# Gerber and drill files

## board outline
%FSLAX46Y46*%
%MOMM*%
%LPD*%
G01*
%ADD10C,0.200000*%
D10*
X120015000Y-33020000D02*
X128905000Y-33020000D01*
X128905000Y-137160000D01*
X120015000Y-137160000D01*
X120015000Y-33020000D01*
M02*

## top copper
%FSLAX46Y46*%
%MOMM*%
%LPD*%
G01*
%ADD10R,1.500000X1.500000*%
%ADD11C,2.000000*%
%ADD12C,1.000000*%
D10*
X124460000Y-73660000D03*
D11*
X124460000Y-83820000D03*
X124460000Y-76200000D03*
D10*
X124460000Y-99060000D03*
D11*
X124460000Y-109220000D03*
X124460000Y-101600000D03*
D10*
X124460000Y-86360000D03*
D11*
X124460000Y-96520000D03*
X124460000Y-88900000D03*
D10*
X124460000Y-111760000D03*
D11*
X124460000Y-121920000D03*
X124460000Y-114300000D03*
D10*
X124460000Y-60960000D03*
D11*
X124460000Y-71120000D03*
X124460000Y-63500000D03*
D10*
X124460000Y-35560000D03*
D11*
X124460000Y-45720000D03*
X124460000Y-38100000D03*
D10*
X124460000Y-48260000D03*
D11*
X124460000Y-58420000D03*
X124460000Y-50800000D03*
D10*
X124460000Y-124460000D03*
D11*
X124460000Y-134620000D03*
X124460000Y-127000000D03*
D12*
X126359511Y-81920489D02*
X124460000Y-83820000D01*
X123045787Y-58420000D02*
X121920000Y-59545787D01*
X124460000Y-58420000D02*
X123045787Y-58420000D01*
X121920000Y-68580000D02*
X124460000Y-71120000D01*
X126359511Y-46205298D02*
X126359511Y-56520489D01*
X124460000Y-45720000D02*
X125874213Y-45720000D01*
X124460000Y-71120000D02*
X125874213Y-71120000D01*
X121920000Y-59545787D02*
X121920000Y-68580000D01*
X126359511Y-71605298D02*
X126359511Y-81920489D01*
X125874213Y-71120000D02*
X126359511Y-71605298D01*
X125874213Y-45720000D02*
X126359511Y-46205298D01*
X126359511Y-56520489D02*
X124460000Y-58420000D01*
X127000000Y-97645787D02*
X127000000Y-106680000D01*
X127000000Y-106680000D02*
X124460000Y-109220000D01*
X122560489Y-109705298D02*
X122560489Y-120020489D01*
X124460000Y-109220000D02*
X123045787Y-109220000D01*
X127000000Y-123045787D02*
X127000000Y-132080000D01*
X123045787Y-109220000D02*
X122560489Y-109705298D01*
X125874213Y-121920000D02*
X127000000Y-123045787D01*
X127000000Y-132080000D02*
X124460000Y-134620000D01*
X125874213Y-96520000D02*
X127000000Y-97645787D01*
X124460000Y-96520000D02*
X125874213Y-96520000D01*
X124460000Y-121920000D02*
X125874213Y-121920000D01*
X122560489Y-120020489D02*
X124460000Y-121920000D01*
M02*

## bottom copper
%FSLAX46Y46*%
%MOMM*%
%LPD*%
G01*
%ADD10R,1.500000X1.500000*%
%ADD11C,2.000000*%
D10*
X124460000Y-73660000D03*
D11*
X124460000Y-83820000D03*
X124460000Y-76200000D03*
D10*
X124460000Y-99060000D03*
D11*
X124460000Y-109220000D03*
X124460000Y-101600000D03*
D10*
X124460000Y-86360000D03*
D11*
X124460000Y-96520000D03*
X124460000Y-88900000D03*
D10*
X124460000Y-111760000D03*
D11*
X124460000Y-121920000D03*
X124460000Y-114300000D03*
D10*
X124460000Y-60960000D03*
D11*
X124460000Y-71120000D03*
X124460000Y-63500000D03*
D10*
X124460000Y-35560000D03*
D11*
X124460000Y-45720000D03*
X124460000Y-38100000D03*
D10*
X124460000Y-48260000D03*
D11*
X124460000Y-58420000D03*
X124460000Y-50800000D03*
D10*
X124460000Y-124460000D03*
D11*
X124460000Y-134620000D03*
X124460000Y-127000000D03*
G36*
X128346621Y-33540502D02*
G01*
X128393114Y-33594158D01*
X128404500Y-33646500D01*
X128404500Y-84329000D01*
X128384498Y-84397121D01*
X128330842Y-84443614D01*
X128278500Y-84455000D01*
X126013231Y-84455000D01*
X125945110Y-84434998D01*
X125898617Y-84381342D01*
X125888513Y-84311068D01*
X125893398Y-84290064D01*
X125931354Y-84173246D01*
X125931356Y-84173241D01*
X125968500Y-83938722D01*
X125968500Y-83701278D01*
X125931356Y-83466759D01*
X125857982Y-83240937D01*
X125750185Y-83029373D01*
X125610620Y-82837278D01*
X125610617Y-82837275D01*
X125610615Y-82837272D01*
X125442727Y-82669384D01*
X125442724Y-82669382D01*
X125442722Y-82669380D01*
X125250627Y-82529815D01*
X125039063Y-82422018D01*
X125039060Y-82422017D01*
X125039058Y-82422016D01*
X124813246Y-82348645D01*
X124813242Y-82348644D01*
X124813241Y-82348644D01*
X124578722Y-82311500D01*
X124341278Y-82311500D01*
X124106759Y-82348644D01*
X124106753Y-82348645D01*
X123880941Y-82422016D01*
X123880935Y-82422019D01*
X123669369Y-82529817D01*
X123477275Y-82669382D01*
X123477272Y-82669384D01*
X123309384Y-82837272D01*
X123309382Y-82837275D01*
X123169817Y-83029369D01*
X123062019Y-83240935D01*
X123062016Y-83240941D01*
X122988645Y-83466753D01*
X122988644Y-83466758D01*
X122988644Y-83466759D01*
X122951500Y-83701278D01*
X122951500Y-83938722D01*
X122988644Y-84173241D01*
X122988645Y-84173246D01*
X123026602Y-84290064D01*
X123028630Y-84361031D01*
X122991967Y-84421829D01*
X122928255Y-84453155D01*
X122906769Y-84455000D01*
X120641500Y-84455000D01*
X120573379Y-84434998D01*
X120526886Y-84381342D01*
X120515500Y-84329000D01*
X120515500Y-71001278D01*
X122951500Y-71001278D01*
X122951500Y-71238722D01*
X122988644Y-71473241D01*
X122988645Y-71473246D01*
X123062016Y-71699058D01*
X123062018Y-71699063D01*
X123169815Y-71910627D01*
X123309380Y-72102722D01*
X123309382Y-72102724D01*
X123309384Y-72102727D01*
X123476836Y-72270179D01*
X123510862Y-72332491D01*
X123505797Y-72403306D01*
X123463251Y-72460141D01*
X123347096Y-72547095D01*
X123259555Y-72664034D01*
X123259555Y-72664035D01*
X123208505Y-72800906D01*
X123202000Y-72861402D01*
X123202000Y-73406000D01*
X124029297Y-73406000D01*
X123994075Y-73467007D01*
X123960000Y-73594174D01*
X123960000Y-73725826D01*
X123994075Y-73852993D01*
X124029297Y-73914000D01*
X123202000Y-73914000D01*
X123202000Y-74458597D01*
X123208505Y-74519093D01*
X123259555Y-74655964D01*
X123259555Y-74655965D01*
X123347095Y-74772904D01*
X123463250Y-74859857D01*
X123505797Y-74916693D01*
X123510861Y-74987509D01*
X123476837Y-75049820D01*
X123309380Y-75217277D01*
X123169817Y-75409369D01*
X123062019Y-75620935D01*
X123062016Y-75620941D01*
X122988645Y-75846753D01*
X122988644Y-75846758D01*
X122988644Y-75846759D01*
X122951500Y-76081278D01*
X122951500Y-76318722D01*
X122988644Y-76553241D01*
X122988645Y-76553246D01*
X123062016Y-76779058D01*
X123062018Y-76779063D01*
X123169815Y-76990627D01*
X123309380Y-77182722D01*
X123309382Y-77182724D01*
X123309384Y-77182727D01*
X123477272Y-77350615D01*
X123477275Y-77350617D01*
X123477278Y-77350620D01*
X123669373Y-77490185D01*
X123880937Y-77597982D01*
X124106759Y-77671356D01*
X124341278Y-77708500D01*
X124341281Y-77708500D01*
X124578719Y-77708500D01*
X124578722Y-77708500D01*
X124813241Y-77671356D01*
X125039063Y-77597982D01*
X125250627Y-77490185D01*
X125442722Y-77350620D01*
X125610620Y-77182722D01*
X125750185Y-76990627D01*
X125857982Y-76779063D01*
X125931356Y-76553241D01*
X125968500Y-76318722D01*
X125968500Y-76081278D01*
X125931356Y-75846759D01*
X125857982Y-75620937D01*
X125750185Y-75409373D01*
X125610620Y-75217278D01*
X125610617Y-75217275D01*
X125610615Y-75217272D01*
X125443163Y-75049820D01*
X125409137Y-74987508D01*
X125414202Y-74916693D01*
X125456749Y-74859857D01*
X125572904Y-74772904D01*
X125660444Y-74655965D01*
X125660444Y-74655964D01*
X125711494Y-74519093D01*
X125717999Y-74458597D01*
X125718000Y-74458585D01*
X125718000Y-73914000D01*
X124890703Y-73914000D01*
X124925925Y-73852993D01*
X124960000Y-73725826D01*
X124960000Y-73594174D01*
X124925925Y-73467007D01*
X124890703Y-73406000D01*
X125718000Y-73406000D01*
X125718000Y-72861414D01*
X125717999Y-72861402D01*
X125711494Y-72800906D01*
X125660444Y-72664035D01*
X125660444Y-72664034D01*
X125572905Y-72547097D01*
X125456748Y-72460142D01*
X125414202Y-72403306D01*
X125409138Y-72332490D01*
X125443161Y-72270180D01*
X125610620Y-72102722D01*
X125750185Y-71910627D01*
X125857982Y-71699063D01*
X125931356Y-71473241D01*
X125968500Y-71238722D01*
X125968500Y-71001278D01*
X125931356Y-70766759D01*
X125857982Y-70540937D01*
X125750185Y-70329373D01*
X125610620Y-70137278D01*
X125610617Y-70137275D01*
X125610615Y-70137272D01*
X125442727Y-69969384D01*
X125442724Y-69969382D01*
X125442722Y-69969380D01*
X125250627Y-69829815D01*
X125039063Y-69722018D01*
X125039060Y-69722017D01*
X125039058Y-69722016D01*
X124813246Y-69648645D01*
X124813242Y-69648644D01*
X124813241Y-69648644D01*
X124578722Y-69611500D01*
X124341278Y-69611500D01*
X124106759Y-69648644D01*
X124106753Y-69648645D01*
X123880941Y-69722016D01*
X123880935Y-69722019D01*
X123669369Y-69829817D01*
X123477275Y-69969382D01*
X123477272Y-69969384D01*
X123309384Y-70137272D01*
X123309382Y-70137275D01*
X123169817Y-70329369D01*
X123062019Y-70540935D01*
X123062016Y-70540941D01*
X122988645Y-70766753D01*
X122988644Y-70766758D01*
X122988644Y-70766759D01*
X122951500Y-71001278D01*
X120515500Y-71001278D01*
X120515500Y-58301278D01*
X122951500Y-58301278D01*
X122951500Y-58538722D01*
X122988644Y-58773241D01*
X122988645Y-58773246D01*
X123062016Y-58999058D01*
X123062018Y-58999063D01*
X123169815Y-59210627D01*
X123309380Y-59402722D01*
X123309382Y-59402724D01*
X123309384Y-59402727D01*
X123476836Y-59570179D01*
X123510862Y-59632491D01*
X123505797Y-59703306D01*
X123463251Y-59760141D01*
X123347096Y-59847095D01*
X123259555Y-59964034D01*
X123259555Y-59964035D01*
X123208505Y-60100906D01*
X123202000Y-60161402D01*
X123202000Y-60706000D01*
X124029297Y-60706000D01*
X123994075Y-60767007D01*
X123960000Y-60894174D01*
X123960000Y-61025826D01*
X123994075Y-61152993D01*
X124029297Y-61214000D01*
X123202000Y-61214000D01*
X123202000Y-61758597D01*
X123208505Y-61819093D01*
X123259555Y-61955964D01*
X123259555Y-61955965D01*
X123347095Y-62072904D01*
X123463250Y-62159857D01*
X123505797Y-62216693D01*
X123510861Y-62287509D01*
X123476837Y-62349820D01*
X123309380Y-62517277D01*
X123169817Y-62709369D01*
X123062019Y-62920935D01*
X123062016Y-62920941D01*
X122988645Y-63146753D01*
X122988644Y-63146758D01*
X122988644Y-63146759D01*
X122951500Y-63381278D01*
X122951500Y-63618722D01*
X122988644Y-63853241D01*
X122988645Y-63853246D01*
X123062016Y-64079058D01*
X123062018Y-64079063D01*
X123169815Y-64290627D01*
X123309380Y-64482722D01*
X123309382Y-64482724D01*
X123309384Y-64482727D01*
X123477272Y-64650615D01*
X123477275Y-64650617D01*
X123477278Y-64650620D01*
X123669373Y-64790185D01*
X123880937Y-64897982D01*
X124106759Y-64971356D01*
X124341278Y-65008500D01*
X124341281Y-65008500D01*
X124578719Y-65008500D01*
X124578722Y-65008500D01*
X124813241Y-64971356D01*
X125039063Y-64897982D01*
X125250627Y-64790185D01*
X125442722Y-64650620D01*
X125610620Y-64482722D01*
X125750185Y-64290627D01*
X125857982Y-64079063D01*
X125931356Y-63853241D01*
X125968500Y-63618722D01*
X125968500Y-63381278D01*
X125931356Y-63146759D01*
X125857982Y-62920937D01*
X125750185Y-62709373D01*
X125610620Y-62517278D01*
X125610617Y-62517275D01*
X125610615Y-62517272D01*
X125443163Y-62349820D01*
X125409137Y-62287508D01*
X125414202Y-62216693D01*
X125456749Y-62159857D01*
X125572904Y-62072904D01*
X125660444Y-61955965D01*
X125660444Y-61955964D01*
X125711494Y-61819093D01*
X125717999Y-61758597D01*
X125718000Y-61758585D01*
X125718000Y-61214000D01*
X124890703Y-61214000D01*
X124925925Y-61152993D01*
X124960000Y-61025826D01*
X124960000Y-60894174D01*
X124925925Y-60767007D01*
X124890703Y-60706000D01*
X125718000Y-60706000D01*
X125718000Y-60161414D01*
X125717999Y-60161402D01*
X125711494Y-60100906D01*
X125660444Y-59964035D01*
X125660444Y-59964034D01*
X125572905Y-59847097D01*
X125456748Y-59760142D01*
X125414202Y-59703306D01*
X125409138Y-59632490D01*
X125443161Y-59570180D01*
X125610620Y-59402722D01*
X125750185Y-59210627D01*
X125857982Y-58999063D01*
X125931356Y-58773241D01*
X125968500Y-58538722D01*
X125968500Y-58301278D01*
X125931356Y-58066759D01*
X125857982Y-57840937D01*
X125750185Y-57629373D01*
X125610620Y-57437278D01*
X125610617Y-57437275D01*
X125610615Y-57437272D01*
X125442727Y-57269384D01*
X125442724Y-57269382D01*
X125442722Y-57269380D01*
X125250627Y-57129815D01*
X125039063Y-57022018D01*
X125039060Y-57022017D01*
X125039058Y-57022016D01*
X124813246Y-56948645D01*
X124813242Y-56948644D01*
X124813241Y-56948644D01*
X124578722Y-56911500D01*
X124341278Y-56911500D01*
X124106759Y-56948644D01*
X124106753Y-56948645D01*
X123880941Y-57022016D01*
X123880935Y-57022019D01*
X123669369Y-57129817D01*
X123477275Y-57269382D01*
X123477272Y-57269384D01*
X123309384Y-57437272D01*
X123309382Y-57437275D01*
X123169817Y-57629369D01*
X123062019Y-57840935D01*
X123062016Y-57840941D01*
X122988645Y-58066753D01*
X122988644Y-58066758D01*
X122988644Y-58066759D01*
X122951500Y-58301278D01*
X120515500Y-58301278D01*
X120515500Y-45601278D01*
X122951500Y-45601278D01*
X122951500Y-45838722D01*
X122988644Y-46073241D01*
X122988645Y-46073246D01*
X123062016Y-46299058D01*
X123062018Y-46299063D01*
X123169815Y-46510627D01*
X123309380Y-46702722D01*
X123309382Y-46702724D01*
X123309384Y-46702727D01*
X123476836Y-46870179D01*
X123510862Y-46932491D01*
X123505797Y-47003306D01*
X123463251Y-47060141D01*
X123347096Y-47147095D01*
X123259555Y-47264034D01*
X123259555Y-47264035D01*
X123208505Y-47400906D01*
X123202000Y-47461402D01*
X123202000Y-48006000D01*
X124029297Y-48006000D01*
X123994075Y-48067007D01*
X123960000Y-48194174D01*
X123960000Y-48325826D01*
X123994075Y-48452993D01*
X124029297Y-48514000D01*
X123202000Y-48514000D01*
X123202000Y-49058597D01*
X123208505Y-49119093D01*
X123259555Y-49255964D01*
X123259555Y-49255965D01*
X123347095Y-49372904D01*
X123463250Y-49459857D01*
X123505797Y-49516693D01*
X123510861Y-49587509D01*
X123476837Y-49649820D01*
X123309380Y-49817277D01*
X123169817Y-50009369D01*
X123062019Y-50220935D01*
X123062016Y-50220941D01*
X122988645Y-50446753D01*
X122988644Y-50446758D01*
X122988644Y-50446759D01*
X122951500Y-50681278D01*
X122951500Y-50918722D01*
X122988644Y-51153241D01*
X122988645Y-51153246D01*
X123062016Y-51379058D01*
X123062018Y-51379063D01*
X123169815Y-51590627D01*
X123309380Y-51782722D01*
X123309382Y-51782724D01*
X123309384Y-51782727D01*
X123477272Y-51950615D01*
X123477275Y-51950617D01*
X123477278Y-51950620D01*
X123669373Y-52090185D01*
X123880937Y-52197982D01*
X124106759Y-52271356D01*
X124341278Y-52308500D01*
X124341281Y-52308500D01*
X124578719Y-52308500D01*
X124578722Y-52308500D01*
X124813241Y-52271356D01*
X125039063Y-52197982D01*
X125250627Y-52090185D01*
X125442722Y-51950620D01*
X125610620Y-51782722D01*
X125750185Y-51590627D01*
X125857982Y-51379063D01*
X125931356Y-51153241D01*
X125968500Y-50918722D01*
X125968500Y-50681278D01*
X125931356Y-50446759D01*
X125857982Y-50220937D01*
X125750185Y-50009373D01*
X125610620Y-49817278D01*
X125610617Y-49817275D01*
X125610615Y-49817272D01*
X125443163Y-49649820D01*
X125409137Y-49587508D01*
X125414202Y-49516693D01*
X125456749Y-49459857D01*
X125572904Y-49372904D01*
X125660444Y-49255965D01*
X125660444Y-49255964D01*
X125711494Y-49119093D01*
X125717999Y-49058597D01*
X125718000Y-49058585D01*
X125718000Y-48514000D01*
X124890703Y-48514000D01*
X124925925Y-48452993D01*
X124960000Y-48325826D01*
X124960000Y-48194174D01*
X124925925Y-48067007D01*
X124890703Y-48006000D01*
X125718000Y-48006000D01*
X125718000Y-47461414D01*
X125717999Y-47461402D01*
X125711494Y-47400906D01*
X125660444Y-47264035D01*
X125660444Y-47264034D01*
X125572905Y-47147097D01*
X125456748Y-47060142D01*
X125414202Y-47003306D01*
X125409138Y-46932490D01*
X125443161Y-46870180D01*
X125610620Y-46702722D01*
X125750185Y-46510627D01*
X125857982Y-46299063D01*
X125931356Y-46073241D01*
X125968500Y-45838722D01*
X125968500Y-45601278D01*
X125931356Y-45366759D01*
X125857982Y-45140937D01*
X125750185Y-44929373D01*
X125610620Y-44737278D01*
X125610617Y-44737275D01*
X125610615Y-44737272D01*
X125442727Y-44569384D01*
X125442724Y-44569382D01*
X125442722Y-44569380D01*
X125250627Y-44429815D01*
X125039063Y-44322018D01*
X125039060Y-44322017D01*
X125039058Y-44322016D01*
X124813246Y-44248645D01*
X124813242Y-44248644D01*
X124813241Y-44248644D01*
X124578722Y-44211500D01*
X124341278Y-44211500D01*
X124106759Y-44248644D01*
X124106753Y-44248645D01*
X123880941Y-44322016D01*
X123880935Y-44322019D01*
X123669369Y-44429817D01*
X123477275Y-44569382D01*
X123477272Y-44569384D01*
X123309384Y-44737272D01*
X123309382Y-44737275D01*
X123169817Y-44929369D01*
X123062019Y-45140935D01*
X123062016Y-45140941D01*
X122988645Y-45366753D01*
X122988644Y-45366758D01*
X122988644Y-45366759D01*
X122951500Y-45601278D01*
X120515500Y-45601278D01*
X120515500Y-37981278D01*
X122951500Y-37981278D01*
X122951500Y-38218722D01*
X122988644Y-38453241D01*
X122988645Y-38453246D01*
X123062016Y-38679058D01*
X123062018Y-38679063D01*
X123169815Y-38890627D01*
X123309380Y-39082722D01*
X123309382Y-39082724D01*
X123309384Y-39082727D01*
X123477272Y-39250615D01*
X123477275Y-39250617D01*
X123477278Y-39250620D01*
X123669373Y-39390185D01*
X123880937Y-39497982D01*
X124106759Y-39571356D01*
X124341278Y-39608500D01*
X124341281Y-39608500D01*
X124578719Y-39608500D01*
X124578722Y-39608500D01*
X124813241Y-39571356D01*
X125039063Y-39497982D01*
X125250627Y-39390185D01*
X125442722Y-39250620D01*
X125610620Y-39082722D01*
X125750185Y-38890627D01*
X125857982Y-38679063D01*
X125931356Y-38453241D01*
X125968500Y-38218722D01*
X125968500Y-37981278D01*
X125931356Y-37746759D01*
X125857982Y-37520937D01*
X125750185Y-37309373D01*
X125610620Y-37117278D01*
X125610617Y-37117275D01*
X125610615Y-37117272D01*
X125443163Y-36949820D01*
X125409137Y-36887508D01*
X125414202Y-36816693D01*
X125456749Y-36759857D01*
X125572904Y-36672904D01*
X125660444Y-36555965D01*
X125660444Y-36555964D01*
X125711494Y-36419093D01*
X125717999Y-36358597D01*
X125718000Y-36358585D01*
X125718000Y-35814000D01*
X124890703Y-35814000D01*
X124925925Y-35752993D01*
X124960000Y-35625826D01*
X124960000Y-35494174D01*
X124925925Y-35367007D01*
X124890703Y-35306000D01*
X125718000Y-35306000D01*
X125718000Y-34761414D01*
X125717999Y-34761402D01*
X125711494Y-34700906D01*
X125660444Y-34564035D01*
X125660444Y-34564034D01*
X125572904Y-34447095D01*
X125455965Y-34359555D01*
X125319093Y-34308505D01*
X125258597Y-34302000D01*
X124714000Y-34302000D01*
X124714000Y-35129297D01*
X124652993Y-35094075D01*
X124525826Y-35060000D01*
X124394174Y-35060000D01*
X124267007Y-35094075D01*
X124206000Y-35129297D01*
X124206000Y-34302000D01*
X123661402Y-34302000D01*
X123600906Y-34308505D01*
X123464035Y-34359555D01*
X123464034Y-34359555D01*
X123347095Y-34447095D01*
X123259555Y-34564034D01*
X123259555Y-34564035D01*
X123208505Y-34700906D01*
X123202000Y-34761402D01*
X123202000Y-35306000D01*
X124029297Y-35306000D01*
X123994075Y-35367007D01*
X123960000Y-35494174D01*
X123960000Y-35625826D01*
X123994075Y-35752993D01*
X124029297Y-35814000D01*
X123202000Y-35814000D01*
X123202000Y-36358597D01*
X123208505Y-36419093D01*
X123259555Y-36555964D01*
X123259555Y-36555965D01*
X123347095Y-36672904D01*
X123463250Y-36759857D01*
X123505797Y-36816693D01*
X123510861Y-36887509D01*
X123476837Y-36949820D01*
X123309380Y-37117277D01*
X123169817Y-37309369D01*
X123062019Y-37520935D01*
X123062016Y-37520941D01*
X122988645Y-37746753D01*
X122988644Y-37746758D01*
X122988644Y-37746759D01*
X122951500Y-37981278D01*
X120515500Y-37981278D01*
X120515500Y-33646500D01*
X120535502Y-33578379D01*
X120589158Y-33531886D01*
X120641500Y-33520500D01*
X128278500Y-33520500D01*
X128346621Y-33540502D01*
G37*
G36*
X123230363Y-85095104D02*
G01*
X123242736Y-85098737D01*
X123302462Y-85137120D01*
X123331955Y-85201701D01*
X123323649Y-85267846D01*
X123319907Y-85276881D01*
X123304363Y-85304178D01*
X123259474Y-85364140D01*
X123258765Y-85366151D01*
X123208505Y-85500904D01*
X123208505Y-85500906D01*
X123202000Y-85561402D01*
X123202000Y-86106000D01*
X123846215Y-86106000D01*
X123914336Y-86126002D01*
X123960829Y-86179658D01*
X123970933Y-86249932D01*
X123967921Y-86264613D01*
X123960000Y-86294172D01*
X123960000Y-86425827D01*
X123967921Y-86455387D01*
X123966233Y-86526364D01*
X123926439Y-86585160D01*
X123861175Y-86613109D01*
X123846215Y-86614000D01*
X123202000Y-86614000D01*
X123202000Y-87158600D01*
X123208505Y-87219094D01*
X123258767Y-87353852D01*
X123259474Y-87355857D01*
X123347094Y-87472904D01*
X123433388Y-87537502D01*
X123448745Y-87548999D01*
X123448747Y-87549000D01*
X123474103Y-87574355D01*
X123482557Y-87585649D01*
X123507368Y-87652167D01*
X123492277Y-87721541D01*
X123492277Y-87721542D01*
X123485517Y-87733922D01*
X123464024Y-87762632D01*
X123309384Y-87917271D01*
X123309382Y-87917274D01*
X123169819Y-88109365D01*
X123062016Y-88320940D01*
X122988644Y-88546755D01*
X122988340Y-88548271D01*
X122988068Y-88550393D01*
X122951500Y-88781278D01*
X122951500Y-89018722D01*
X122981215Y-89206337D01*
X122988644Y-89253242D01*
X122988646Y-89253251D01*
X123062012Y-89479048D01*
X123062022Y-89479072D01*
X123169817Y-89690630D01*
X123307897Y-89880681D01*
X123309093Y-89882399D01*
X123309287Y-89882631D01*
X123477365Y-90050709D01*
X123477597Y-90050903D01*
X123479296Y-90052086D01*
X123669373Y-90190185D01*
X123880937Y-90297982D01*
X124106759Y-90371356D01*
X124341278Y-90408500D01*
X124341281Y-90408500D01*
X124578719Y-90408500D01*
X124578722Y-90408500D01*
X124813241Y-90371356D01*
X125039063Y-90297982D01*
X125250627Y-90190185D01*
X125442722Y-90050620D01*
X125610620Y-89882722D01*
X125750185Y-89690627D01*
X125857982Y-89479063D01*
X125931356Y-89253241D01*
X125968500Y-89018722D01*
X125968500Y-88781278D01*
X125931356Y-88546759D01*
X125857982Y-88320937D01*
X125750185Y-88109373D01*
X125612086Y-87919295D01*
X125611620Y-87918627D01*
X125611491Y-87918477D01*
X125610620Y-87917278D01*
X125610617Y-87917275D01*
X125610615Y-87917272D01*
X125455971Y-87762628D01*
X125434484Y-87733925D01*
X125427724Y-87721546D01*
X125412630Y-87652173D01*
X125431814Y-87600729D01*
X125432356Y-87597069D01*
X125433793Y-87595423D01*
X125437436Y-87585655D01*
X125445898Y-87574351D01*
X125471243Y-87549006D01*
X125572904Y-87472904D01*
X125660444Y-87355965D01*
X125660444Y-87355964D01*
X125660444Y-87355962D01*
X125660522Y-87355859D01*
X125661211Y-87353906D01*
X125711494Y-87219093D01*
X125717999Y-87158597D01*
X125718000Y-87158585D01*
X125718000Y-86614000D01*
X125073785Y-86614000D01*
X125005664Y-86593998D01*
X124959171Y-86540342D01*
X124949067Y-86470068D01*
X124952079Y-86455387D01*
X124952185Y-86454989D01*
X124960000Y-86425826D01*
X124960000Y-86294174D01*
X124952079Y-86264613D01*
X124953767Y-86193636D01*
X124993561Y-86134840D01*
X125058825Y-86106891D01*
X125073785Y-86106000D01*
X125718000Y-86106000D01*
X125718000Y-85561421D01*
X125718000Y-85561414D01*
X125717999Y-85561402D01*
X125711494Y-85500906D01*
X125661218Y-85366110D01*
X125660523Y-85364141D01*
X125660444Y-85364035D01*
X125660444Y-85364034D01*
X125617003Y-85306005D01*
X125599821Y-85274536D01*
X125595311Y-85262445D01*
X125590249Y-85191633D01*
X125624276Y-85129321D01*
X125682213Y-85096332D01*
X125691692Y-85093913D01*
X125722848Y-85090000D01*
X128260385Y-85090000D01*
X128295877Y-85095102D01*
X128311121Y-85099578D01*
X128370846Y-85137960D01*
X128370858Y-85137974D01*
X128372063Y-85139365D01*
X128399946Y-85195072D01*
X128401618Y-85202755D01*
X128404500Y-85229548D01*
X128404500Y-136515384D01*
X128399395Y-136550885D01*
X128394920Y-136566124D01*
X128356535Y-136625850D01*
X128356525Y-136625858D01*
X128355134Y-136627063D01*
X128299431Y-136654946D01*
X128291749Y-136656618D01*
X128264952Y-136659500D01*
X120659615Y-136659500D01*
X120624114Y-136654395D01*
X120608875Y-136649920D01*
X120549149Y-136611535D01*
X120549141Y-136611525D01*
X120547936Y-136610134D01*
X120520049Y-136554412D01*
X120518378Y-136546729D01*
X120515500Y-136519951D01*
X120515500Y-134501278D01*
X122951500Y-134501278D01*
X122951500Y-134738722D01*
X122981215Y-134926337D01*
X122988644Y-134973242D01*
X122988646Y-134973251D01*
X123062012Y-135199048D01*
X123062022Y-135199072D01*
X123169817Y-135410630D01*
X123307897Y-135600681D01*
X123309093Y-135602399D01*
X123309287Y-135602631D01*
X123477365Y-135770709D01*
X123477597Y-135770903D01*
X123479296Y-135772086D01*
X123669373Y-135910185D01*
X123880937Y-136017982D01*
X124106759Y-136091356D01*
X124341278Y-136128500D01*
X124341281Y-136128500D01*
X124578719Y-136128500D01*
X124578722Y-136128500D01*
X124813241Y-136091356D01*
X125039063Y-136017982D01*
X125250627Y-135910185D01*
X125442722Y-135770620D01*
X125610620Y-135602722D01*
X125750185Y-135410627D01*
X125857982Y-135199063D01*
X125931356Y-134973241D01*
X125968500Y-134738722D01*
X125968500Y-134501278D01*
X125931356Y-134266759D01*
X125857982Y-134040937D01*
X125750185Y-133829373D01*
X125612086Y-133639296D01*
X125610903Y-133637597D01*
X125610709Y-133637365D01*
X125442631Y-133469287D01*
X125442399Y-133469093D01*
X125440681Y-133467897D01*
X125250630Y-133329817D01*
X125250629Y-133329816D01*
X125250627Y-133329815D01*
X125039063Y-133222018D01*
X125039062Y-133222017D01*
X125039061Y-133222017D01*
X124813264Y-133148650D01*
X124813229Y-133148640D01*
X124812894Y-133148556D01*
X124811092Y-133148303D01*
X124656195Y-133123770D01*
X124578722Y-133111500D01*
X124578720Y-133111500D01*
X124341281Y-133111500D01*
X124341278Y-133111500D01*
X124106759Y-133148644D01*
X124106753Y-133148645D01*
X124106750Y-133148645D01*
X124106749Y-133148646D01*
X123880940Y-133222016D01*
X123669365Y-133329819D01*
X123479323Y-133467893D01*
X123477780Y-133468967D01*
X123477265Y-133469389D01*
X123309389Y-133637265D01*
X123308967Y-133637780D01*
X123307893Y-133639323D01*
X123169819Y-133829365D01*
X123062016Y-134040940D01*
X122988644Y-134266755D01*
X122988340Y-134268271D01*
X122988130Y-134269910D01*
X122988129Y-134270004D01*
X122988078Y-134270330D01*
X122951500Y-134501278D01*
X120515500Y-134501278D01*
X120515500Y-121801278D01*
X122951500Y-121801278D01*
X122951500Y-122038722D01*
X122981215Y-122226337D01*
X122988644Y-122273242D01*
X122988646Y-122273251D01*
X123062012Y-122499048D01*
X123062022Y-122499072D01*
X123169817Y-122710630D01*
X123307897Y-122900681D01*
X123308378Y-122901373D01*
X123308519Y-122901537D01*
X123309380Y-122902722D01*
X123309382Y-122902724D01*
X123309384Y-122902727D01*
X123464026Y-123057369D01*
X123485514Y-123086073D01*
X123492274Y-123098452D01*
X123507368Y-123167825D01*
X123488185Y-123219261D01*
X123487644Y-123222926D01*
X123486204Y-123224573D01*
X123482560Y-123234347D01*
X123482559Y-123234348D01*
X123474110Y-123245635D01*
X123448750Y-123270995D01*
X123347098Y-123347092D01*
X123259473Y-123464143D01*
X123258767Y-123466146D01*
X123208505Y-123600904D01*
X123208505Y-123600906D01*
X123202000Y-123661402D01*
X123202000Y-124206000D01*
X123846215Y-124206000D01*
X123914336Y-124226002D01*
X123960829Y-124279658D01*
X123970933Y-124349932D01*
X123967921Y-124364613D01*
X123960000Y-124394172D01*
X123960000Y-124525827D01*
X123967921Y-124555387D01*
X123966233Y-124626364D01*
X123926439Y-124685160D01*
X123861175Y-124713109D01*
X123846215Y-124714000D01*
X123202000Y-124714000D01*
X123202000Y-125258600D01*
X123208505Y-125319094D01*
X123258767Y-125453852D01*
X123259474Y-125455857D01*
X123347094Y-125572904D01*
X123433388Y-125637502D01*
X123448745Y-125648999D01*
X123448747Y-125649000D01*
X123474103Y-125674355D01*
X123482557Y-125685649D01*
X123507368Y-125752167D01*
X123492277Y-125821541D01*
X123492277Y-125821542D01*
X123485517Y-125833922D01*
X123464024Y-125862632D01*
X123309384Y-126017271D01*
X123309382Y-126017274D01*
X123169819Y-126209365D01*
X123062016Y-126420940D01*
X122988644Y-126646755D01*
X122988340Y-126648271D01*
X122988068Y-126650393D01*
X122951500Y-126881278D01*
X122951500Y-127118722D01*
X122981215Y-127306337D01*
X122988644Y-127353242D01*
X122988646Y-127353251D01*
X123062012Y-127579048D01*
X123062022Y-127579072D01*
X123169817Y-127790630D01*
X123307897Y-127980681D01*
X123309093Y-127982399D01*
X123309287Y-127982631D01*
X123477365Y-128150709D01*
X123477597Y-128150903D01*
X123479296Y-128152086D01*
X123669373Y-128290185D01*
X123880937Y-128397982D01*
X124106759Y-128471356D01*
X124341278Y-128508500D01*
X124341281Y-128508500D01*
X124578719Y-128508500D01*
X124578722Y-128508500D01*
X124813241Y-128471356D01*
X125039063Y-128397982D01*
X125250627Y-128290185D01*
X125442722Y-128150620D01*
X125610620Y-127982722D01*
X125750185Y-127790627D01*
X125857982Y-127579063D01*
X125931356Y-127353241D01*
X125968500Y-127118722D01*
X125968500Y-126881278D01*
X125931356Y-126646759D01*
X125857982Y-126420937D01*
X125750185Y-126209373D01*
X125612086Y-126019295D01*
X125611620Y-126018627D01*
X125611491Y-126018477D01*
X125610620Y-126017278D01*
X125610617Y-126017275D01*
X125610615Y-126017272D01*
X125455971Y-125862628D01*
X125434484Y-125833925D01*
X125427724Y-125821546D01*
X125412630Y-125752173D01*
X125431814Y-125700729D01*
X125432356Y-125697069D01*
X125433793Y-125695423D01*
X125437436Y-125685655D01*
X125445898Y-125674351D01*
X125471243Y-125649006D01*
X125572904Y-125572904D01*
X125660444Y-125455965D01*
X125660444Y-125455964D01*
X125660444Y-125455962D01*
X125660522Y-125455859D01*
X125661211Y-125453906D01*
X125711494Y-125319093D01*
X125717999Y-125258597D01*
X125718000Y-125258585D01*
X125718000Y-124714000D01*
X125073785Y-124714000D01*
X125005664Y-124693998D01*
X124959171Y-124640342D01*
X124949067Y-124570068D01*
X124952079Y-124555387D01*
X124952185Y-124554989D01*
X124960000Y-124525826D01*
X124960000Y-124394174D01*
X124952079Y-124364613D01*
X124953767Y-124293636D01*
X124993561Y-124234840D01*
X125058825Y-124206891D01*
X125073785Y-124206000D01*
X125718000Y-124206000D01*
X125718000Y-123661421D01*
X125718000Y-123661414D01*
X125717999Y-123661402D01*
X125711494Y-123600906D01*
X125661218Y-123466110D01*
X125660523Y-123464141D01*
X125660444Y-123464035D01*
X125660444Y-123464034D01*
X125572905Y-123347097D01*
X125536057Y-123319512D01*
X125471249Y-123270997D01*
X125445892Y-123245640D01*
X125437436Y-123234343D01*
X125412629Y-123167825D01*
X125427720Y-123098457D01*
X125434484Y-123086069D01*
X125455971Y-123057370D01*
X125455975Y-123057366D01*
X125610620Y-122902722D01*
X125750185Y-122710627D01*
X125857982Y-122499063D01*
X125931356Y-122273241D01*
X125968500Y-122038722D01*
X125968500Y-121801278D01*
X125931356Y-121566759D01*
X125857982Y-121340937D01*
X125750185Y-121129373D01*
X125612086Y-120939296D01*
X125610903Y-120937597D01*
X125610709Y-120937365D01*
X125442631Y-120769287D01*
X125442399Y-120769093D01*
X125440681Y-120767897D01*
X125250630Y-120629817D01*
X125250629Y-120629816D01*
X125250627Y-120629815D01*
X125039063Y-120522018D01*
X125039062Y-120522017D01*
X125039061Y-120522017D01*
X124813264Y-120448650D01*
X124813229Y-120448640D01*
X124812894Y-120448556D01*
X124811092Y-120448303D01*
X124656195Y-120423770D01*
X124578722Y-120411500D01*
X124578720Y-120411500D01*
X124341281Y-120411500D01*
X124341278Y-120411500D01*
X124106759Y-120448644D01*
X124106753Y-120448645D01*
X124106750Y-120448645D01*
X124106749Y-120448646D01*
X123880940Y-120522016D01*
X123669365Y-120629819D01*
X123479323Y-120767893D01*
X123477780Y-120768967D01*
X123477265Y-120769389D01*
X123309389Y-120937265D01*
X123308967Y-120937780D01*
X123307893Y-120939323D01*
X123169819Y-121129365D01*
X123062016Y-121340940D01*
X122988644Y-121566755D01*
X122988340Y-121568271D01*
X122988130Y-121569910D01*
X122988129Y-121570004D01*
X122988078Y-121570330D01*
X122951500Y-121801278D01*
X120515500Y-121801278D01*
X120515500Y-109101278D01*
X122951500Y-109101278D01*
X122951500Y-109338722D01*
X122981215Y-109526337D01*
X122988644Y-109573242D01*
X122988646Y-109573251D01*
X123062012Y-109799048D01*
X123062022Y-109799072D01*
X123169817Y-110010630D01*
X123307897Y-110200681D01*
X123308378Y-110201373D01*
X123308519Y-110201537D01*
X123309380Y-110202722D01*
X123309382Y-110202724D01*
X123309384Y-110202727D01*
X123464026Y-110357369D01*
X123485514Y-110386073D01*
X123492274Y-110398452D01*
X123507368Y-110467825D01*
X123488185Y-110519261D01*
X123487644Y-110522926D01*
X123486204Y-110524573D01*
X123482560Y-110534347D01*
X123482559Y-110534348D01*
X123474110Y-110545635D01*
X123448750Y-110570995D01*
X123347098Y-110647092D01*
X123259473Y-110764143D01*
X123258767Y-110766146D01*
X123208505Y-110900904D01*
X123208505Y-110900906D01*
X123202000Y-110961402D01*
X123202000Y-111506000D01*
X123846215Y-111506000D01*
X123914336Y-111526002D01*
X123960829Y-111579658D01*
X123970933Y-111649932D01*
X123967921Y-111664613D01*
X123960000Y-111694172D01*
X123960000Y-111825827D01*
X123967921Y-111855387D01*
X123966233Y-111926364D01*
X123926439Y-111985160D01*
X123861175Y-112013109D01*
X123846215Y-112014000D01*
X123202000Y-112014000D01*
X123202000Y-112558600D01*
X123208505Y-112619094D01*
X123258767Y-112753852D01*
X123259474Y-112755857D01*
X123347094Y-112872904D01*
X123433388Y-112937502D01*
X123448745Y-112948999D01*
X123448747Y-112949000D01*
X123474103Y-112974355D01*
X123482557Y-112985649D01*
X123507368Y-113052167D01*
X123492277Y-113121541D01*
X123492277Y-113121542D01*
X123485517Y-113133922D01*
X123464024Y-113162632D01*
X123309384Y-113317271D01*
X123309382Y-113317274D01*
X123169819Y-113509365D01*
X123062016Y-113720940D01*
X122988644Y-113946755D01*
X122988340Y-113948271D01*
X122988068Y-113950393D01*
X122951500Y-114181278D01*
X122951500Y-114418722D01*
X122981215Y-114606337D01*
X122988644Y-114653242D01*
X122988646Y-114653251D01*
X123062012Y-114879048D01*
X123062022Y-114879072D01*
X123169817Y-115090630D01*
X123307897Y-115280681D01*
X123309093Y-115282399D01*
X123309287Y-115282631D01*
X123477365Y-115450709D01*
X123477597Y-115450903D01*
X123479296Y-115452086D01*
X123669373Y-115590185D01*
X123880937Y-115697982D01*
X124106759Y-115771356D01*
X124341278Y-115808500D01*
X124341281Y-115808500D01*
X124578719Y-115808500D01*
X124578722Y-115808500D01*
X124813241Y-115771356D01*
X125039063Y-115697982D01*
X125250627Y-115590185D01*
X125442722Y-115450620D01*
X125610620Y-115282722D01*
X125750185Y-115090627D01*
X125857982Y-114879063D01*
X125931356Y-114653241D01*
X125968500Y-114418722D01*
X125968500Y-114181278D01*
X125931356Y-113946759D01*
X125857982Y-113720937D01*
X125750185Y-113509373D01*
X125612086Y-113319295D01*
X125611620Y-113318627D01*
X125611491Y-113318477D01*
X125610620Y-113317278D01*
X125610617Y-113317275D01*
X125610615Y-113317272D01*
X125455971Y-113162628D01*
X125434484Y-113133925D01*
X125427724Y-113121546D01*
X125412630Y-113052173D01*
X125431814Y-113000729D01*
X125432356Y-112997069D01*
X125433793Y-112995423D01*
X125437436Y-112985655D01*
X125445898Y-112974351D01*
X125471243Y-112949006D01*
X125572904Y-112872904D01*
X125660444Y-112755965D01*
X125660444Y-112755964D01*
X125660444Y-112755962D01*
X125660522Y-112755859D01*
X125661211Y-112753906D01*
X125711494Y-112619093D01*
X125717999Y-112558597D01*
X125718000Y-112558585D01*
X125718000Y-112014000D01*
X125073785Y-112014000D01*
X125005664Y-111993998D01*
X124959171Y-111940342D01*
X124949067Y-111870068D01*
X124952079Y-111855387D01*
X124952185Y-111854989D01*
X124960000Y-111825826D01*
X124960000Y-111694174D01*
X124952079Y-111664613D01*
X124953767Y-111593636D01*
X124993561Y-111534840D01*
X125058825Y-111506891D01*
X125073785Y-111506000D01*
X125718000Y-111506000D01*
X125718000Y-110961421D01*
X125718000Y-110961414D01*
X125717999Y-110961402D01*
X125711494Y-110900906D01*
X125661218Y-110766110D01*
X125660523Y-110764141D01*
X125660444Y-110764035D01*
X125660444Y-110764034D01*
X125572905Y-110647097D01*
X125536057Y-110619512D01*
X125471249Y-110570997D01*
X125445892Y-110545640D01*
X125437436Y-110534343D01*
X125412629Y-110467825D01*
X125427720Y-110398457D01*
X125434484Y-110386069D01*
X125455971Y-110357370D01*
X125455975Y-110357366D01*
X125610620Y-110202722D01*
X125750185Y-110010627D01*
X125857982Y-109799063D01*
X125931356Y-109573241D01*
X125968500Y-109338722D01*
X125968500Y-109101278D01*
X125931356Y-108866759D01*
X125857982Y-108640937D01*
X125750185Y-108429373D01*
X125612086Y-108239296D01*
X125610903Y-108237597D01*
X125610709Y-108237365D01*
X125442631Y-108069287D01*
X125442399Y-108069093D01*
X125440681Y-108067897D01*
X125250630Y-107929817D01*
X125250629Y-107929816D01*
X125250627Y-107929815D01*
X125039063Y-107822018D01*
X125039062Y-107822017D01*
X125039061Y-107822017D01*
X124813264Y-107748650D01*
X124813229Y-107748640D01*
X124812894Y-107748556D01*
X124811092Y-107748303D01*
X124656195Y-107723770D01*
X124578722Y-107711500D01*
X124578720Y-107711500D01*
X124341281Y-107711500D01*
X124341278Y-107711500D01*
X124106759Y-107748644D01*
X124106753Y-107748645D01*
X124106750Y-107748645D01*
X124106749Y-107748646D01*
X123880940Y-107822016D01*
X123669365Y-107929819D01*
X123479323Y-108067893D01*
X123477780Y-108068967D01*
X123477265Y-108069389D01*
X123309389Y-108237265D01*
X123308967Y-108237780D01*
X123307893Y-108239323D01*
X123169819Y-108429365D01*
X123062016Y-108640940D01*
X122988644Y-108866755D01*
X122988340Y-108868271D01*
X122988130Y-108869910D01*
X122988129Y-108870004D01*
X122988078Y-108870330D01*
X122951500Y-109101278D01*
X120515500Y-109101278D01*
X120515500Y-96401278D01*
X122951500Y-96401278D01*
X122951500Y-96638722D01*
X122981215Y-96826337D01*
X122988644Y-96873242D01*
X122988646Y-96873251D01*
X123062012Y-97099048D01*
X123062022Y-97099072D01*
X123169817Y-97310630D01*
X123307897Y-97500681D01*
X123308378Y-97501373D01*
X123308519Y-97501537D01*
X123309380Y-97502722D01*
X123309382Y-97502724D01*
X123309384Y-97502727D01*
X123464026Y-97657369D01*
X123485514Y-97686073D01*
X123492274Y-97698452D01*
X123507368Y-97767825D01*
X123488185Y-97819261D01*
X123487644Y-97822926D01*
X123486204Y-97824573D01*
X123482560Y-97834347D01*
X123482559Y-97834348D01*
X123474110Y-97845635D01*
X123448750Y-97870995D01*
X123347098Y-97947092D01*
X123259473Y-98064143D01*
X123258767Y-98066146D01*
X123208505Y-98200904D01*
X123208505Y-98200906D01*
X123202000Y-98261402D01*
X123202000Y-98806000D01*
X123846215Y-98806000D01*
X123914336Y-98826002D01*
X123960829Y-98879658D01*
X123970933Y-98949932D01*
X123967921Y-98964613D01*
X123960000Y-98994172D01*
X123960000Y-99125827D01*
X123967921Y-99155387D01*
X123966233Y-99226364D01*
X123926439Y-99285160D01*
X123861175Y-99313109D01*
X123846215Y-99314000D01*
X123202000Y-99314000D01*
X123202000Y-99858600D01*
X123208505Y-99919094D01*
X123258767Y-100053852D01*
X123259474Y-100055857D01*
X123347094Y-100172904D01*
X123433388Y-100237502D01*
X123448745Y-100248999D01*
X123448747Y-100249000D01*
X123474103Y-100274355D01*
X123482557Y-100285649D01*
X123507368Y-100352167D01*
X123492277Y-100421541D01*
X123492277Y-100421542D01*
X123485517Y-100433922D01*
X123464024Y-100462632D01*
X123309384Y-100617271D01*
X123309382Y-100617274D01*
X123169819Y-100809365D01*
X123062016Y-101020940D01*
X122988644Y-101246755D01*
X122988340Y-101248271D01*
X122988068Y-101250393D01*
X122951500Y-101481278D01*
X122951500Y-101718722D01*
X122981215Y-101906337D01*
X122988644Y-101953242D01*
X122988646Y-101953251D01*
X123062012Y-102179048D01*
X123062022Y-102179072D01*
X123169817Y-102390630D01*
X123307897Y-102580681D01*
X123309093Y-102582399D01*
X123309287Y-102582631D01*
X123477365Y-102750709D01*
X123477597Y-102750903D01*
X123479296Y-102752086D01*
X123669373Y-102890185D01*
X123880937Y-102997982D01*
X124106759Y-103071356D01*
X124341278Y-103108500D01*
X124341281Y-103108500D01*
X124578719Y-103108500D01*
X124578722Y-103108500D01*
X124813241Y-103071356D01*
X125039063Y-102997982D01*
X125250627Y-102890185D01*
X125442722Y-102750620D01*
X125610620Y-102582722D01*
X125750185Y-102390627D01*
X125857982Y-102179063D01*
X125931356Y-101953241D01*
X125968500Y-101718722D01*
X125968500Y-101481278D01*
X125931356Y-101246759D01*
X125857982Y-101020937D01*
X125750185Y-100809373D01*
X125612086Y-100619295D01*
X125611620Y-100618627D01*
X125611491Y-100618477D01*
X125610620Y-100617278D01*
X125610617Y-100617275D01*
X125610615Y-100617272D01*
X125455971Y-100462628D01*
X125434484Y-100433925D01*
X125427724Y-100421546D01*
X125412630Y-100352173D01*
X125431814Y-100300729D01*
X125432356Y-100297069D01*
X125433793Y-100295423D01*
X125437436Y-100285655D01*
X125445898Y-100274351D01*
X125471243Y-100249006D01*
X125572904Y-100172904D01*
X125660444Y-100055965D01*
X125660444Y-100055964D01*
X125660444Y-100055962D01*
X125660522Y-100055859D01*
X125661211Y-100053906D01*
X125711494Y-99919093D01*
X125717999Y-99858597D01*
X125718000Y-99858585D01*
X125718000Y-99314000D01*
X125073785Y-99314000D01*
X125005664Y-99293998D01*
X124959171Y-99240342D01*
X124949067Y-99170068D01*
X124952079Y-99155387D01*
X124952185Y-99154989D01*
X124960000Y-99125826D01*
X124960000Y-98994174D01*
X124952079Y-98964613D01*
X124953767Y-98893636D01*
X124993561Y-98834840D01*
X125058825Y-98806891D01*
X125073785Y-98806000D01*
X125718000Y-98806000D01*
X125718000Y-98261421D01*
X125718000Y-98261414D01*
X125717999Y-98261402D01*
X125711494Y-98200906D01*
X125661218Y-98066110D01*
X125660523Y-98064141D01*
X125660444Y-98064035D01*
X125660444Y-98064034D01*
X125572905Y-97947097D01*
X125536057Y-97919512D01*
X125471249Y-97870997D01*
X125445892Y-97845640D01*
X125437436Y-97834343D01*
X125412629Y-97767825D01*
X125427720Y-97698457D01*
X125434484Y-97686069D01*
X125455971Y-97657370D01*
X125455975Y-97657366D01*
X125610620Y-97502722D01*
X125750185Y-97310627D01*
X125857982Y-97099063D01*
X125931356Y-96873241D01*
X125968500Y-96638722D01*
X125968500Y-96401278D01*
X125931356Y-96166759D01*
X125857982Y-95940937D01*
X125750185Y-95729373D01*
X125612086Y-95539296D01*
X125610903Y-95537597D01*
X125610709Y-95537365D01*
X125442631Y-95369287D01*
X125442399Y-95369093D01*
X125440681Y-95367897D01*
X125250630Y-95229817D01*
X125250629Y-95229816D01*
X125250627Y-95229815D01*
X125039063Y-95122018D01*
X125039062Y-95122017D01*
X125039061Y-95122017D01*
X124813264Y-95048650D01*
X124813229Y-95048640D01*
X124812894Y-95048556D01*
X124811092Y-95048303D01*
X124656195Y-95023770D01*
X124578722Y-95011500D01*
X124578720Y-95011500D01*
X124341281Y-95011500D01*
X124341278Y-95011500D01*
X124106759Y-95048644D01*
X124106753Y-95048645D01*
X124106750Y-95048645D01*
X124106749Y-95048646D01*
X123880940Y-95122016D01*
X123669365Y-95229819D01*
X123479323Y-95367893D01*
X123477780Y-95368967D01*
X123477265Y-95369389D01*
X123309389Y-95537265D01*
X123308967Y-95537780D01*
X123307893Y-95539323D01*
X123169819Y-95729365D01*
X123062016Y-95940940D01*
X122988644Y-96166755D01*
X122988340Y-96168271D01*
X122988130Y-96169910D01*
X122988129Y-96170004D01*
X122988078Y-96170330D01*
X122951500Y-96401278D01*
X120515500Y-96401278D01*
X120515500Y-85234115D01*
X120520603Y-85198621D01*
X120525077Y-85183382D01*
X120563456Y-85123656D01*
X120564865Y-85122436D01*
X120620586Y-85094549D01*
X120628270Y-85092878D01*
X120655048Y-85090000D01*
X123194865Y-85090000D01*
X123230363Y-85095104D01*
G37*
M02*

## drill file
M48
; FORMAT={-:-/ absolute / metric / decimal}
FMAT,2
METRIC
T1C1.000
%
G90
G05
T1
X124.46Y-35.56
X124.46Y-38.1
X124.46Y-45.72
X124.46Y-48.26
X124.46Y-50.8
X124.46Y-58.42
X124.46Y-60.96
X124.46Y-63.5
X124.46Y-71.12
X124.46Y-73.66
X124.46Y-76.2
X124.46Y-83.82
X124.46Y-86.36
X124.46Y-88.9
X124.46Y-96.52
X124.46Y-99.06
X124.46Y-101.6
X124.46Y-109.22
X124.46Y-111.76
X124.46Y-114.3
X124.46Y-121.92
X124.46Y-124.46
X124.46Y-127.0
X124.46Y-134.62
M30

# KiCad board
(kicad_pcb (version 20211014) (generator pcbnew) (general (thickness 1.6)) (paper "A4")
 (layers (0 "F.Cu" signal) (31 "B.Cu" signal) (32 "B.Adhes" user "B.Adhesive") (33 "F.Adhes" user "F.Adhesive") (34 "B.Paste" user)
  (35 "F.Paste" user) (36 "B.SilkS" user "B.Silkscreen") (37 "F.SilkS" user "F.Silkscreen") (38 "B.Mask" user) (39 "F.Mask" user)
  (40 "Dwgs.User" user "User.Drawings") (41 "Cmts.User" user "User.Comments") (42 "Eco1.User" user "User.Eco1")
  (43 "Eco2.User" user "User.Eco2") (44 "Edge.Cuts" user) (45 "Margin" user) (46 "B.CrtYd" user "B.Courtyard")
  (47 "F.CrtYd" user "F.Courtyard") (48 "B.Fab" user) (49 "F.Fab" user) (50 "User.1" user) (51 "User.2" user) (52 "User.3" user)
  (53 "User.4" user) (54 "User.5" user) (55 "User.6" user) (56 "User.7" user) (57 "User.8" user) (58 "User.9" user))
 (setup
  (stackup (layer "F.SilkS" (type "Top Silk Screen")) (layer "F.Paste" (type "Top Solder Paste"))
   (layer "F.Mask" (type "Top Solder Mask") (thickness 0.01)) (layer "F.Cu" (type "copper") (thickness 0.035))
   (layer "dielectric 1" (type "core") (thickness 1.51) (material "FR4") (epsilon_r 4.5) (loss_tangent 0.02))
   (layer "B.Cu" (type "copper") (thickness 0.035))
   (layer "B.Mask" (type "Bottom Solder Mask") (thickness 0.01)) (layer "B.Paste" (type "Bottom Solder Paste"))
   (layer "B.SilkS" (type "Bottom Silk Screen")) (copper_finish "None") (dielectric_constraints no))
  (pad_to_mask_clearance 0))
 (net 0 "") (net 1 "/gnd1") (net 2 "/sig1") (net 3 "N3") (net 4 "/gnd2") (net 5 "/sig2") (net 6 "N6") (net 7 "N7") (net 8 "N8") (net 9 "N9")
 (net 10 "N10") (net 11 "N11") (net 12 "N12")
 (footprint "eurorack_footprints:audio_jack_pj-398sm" (layer "F.Cu") (at 124.46 83.82)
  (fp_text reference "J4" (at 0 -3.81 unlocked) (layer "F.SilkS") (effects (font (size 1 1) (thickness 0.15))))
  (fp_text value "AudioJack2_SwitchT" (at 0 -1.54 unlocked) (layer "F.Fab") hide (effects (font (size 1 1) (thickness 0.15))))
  (pad "S" thru_hole rect (at 0 -10.16) (size 1.5 1.5) (drill 1) (layers *.Cu *.Mask) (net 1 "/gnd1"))
  (pad "T" thru_hole circle (at 0 0) (size 2 2) (drill 1) (layers *.Cu *.Mask) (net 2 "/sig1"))
  (pad "TN" thru_hole circle (at 0 -7.62) (size 2 2) (drill 1) (layers *.Cu *.Mask) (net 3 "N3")))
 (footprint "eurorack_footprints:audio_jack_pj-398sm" (layer "F.Cu") (at 124.46 109.22)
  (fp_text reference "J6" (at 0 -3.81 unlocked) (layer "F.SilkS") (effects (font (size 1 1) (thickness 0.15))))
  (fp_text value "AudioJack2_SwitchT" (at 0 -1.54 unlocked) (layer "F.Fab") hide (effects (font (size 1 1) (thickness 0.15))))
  (pad "S" thru_hole rect (at 0 -10.16) (size 1.5 1.5) (drill 1) (layers *.Cu *.Mask) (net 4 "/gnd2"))
  (pad "T" thru_hole circle (at 0 0) (size 2 2) (drill 1) (layers *.Cu *.Mask) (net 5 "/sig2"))
  (pad "TN" thru_hole circle (at 0 -7.62) (size 2 2) (drill 1) (layers *.Cu *.Mask) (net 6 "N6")))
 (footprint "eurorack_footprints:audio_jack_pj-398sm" (layer "F.Cu") (at 124.46 96.52)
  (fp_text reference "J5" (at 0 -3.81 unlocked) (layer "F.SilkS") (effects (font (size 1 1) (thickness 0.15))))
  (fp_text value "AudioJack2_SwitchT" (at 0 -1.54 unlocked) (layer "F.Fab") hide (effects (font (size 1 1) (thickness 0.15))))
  (pad "S" thru_hole rect (at 0 -10.16) (size 1.5 1.5) (drill 1) (layers *.Cu *.Mask) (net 4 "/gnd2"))
  (pad "T" thru_hole circle (at 0 0) (size 2 2) (drill 1) (layers *.Cu *.Mask) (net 5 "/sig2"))
  (pad "TN" thru_hole circle (at 0 -7.62) (size 2 2) (drill 1) (layers *.Cu *.Mask) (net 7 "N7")))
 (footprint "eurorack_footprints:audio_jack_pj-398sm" (layer "F.Cu") (at 124.46 121.92)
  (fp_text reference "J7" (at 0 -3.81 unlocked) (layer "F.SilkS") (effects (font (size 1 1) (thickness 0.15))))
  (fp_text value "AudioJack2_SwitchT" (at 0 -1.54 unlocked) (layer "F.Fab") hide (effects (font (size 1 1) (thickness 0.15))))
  (pad "S" thru_hole rect (at 0 -10.16) (size 1.5 1.5) (drill 1) (layers *.Cu *.Mask) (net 4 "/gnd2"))
  (pad "T" thru_hole circle (at 0 0) (size 2 2) (drill 1) (layers *.Cu *.Mask) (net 5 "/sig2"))
  (pad "TN" thru_hole circle (at 0 -7.62) (size 2 2) (drill 1) (layers *.Cu *.Mask) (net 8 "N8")))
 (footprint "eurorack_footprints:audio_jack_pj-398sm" (layer "F.Cu") (at 124.46 71.12)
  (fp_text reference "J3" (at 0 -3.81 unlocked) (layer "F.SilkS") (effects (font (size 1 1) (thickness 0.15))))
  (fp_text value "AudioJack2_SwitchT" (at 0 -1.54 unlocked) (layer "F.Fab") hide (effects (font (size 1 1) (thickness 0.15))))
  (pad "S" thru_hole rect (at 0 -10.16) (size 1.5 1.5) (drill 1) (layers *.Cu *.Mask) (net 1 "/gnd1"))
  (pad "T" thru_hole circle (at 0 0) (size 2 2) (drill 1) (layers *.Cu *.Mask) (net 2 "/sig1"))
  (pad "TN" thru_hole circle (at 0 -7.62) (size 2 2) (drill 1) (layers *.Cu *.Mask) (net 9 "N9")))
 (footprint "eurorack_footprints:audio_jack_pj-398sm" (layer "F.Cu") (at 124.46 45.72)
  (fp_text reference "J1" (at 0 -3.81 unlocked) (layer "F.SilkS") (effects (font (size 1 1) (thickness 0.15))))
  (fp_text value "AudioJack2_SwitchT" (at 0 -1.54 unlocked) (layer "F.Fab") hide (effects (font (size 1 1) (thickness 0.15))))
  (pad "S" thru_hole rect (at 0 -10.16) (size 1.5 1.5) (drill 1) (layers *.Cu *.Mask) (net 1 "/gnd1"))
  (pad "T" thru_hole circle (at 0 0) (size 2 2) (drill 1) (layers *.Cu *.Mask) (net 2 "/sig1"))
  (pad "TN" thru_hole circle (at 0 -7.62) (size 2 2) (drill 1) (layers *.Cu *.Mask) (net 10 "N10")))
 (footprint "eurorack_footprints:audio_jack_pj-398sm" (layer "F.Cu") (at 124.46 58.42)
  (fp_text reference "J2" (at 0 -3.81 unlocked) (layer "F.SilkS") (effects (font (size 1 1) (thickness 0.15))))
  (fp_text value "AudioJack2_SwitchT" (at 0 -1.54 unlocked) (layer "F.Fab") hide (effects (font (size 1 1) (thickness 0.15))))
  (pad "S" thru_hole rect (at 0 -10.16) (size 1.5 1.5) (drill 1) (layers *.Cu *.Mask) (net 1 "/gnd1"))
  (pad "T" thru_hole circle (at 0 0) (size 2 2) (drill 1) (layers *.Cu *.Mask) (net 2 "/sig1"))
  (pad "TN" thru_hole circle (at 0 -7.62) (size 2 2) (drill 1) (layers *.Cu *.Mask) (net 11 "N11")))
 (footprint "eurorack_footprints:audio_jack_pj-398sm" (layer "F.Cu") (at 124.46 134.62)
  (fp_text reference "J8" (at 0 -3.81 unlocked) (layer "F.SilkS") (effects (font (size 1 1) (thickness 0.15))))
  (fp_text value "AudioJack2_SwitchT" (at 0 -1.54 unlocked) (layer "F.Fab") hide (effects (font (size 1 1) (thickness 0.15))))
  (pad "S" thru_hole rect (at 0 -10.16) (size 1.5 1.5) (drill 1) (layers *.Cu *.Mask) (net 4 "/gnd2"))
  (pad "T" thru_hole circle (at 0 0) (size 2 2) (drill 1) (layers *.Cu *.Mask) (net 5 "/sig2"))
  (pad "TN" thru_hole circle (at 0 -7.62) (size 2 2) (drill 1) (layers *.Cu *.Mask) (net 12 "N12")))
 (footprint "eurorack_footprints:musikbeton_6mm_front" (layer "B.Cu") (at 124.46 130.81 180)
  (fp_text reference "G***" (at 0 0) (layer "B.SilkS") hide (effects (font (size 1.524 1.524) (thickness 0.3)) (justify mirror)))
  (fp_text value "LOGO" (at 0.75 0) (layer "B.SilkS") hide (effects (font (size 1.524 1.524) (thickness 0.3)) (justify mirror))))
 (gr_rect (start 120.015 137.16) (end 128.905 33.02) (layer "Edge.Cuts") (width 0.2) (fill none))
 (segment (start 126.359511 81.920489) (end 124.46 83.82) (width 1) (layer "F.Cu") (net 2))
 (segment (start 123.045787 58.42) (end 121.92 59.545787) (width 1) (layer "F.Cu") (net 2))
 (segment (start 124.46 58.42) (end 123.045787 58.42) (width 1) (layer "F.Cu") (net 2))
 (segment (start 121.92 68.58) (end 124.46 71.12) (width 1) (layer "F.Cu") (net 2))
 (segment (start 126.359511 46.205298) (end 126.359511 56.520489) (width 1) (layer "F.Cu") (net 2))
 (segment (start 124.46 45.72) (end 125.874213 45.72) (width 1) (layer "F.Cu") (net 2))
 (segment (start 124.46 71.12) (end 125.874213 71.12) (width 1) (layer "F.Cu") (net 2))
 (segment (start 121.92 59.545787) (end 121.92 68.58) (width 1) (layer "F.Cu") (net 2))
 (segment (start 126.359511 71.605298) (end 126.359511 81.920489) (width 1) (layer "F.Cu") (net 2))
 (segment (start 125.874213 71.12) (end 126.359511 71.605298) (width 1) (layer "F.Cu") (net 2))
 (segment (start 125.874213 45.72) (end 126.359511 46.205298) (width 1) (layer "F.Cu") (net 2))
 (segment (start 126.359511 56.520489) (end 124.46 58.42) (width 1) (layer "F.Cu") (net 2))
 (segment (start 127 97.645787) (end 127 106.68) (width 1) (layer "F.Cu") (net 5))
 (segment (start 127 106.68) (end 124.46 109.22) (width 1) (layer "F.Cu") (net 5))
 (segment (start 122.560489 109.705298) (end 122.560489 120.020489) (width 1) (layer "F.Cu") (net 5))
 (segment (start 124.46 109.22) (end 123.045787 109.22) (width 1) (layer "F.Cu") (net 5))
 (segment (start 127 123.045787) (end 127 132.08) (width 1) (layer "F.Cu") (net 5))
 (segment (start 123.045787 109.22) (end 122.560489 109.705298) (width 1) (layer "F.Cu") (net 5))
 (segment (start 125.874213 121.92) (end 127 123.045787) (width 1) (layer "F.Cu") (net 5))
 (segment (start 127 132.08) (end 124.46 134.62) (width 1) (layer "F.Cu") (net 5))
 (segment (start 125.874213 96.52) (end 127 97.645787) (width 1) (layer "F.Cu") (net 5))
 (segment (start 124.46 96.52) (end 125.874213 96.52) (width 1) (layer "F.Cu") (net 5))
 (segment (start 124.46 121.92) (end 125.874213 121.92) (width 1) (layer "F.Cu") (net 5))
 (segment (start 122.560489 120.020489) (end 124.46 121.92) (width 1) (layer "F.Cu") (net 5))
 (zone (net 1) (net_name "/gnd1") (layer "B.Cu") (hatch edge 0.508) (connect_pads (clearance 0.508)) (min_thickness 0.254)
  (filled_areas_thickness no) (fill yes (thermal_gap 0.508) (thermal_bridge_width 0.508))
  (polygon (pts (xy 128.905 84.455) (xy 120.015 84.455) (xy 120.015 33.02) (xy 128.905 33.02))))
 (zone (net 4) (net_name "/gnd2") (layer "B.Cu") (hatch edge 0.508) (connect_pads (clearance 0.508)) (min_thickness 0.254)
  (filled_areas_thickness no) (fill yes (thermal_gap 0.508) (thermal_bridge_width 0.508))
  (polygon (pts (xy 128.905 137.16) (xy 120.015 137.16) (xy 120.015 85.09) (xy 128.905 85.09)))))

